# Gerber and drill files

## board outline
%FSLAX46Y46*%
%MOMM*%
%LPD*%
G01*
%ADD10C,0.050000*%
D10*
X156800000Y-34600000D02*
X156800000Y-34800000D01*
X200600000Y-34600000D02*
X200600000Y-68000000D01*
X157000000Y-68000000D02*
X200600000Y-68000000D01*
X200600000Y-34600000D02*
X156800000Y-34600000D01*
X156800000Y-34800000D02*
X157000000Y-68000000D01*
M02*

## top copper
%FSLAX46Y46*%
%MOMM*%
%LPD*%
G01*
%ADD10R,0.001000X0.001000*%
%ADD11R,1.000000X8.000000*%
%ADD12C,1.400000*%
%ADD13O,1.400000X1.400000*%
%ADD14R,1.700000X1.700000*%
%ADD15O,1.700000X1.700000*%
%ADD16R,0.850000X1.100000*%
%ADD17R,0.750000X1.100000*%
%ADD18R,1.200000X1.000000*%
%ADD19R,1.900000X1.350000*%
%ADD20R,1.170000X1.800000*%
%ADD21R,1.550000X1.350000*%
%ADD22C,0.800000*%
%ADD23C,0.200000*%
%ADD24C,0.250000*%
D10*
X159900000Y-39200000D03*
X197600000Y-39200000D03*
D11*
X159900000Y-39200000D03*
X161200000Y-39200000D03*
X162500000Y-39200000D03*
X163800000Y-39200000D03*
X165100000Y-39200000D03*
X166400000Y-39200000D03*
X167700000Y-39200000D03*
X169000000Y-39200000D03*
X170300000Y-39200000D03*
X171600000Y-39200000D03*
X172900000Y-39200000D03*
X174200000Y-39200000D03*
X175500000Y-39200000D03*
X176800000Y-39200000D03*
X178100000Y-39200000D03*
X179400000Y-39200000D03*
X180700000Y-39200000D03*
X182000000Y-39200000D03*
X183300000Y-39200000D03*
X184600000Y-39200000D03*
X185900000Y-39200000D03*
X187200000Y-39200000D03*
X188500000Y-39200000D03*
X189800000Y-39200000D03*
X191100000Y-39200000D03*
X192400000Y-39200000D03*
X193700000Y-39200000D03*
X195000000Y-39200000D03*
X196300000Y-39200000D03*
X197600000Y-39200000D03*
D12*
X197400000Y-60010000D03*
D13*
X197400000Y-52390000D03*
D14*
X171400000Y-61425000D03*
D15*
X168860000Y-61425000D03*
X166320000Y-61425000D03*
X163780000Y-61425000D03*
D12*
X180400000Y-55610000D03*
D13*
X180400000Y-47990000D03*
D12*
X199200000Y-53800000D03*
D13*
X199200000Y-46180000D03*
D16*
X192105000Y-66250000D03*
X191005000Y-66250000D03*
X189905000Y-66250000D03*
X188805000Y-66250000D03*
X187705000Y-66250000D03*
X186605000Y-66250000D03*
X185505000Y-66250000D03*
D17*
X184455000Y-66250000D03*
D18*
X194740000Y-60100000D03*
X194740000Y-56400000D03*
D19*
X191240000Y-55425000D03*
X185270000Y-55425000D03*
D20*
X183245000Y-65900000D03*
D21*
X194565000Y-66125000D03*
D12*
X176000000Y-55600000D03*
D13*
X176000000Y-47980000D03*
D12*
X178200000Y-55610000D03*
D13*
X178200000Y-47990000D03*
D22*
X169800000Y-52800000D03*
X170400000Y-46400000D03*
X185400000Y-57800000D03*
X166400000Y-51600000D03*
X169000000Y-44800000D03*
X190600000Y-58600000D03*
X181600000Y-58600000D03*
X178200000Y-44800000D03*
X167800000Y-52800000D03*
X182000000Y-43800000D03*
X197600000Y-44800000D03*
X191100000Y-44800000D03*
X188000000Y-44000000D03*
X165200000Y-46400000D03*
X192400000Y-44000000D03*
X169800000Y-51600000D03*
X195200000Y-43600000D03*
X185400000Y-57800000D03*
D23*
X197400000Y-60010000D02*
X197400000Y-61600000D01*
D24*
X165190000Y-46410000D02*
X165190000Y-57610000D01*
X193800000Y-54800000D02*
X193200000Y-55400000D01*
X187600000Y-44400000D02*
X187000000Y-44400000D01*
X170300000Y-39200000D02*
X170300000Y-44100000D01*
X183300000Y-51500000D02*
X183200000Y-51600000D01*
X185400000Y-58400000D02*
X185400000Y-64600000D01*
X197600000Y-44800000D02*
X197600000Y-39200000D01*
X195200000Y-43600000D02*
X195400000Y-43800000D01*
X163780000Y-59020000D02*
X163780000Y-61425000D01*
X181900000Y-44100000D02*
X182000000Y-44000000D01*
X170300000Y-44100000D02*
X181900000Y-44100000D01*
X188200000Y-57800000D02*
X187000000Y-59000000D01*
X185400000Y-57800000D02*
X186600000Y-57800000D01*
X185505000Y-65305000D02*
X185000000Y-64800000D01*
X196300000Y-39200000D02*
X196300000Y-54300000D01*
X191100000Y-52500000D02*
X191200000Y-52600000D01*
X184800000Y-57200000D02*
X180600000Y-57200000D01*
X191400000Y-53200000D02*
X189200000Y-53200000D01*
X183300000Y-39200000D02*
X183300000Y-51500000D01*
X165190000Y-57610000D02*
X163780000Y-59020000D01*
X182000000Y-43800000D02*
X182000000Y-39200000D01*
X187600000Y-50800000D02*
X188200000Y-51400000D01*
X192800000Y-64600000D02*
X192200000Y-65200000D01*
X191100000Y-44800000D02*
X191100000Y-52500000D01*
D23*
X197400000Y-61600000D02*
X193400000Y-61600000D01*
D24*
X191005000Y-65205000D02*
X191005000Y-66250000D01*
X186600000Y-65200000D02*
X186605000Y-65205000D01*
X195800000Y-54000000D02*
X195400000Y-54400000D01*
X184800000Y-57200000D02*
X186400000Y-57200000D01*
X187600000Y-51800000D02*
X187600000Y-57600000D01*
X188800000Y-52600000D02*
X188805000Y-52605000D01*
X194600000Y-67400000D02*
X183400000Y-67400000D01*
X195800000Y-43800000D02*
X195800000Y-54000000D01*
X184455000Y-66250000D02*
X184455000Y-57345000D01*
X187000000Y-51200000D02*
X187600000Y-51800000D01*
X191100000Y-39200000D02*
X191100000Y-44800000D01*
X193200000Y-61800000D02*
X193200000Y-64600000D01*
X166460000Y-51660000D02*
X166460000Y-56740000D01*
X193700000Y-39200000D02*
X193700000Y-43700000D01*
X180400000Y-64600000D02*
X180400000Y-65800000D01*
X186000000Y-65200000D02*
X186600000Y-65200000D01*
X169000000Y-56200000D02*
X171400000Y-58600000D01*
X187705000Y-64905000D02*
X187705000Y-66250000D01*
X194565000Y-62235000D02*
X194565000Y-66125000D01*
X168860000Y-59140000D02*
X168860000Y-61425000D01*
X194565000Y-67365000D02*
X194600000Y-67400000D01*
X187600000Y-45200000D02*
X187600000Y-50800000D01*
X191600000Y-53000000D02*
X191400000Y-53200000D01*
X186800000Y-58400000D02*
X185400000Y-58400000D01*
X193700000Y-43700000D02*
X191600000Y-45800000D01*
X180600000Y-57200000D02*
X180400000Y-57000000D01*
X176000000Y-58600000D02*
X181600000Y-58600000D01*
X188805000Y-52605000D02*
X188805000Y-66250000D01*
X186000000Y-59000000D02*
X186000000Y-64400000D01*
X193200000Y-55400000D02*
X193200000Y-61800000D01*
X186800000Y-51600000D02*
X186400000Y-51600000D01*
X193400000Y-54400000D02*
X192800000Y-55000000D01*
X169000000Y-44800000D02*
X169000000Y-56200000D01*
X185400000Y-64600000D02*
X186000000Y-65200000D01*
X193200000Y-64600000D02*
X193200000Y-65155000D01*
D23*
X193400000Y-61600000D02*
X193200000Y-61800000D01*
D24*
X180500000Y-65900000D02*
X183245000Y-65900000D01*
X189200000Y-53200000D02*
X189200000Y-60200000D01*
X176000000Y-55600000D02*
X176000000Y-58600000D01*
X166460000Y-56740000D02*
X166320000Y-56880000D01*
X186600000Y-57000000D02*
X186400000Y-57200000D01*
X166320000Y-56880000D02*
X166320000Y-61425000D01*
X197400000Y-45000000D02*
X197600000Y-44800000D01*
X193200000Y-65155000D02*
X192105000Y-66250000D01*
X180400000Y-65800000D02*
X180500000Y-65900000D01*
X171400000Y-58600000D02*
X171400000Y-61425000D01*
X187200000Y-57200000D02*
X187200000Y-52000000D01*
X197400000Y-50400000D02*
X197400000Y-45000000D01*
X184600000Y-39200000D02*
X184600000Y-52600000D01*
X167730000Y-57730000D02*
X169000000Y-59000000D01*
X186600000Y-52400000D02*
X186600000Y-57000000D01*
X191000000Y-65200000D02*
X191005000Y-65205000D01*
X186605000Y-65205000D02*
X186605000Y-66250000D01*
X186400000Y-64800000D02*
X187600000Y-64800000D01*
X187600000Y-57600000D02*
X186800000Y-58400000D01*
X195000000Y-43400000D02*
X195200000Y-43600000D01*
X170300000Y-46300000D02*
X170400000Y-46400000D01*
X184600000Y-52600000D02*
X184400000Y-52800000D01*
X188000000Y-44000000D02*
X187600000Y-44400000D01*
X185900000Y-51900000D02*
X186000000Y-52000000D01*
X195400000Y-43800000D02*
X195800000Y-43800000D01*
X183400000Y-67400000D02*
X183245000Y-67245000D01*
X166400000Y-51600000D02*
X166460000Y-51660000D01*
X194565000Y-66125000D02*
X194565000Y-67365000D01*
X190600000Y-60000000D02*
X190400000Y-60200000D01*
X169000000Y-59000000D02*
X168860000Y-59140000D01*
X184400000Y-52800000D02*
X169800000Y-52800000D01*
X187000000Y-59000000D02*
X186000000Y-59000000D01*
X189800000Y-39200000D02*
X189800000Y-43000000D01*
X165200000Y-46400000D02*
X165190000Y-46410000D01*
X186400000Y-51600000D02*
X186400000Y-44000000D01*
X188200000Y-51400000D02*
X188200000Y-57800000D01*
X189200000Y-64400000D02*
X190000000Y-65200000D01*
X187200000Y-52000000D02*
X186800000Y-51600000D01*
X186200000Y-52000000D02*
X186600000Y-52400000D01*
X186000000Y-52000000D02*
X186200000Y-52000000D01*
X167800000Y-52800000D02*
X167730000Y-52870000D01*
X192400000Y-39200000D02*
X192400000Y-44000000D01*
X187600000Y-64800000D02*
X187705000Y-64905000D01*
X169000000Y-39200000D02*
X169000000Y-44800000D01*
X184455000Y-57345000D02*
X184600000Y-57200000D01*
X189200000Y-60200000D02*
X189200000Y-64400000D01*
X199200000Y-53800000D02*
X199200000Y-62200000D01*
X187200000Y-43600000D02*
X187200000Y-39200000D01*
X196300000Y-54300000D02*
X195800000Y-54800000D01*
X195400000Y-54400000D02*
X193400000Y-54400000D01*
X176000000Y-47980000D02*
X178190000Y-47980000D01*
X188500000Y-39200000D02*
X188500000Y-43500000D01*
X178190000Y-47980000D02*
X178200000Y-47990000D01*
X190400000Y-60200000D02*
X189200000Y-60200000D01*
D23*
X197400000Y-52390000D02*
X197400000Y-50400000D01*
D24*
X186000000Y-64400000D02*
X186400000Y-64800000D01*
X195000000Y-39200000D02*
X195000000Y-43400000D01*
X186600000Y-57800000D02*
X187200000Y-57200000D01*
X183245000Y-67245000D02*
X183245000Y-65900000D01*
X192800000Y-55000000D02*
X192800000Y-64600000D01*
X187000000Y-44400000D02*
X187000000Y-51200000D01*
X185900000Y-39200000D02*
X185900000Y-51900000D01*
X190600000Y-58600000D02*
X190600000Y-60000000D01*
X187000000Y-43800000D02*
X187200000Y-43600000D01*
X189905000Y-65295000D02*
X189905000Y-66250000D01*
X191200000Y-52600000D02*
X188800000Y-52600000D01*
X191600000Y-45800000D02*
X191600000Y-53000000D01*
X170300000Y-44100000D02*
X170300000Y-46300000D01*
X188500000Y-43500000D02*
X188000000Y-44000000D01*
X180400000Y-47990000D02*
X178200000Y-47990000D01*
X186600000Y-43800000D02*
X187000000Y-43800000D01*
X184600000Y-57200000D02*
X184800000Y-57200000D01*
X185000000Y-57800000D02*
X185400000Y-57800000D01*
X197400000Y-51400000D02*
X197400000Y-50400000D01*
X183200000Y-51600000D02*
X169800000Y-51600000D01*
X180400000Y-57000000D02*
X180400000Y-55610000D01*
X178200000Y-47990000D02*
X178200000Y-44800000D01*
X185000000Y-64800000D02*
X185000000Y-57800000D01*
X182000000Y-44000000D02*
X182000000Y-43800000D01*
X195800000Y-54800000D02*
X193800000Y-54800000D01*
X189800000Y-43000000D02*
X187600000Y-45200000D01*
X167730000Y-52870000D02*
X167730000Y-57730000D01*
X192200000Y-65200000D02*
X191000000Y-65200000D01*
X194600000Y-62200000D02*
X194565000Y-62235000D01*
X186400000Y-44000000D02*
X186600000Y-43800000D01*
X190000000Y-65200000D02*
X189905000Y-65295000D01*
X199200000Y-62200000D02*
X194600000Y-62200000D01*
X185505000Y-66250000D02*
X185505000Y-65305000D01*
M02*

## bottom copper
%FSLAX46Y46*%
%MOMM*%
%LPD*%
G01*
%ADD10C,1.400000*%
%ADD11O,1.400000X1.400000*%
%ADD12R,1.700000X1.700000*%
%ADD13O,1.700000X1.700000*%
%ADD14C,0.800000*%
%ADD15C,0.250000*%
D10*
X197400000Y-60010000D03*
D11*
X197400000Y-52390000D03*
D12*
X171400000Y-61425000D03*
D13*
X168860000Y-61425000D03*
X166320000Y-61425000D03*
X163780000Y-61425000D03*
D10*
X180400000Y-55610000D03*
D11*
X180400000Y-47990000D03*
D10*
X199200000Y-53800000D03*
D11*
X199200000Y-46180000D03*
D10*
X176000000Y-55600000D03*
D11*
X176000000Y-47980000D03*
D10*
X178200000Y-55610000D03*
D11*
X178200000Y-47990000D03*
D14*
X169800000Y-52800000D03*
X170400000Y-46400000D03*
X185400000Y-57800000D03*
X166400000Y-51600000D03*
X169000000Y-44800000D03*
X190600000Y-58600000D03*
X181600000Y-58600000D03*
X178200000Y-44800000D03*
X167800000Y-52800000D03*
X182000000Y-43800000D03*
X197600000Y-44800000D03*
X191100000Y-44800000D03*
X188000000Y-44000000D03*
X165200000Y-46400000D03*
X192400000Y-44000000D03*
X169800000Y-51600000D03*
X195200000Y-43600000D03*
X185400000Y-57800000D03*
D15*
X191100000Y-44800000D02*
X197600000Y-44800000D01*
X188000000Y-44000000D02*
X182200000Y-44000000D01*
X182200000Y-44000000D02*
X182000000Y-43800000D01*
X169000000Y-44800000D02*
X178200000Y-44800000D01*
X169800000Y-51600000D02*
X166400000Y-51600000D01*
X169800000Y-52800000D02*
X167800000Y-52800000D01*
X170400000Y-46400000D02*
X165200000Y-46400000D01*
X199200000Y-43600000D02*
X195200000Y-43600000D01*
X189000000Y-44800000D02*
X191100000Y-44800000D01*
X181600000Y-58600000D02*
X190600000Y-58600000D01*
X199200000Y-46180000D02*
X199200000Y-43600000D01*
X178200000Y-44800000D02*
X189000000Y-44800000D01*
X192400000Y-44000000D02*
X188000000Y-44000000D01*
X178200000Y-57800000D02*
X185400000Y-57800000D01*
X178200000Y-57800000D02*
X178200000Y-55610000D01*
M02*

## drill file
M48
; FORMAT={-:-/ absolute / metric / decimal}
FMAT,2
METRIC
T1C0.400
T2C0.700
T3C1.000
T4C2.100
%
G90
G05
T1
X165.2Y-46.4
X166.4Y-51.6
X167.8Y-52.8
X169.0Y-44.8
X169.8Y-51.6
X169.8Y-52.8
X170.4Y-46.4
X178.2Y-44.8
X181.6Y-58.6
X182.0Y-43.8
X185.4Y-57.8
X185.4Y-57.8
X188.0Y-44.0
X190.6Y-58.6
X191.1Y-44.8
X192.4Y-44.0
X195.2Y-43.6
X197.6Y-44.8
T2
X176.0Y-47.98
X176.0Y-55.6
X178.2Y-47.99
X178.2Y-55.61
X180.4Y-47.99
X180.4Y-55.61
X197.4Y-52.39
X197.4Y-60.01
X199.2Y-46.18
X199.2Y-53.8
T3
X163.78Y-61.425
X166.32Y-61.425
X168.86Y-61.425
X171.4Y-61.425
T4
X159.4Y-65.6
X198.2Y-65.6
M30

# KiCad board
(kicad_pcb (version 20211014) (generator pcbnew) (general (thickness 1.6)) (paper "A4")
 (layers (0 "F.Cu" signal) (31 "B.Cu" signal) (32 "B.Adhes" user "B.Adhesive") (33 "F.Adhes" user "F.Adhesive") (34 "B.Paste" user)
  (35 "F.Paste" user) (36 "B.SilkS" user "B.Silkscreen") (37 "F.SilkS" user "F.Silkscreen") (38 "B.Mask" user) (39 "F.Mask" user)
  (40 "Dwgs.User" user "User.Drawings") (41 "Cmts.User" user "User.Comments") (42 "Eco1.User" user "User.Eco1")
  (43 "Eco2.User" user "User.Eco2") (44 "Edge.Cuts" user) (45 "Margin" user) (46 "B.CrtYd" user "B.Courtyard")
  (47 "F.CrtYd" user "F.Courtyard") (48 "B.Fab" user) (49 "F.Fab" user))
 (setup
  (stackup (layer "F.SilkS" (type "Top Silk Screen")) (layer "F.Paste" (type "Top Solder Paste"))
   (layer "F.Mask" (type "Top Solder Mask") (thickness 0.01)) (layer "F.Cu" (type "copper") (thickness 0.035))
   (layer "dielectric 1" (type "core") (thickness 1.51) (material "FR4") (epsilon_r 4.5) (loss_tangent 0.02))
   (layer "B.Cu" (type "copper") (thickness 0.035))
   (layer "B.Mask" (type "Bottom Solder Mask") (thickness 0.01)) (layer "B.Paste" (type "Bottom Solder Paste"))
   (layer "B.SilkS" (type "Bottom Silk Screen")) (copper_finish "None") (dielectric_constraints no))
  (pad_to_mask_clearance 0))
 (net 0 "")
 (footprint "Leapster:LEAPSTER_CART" (layer "F.Cu") (at 178.75 39.2)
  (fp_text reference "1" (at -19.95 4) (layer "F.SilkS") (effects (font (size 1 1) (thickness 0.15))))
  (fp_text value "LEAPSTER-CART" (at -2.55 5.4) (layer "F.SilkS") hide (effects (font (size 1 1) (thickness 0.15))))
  (pad "0" smd rect locked (at -18.85 0) (size 0.001 0.001) (layers "F.Cu" "F.Paste" "F.Mask"))
  (pad "0" smd rect locked (at 18.85 0) (size 0.001 0.001) (layers "F.Cu" "F.Paste" "F.Mask"))
  (pad "1" connect rect locked (at -18.85 0) (size 1 8) (layers "F.Cu" "F.Mask"))
  (pad "2" connect rect locked (at -17.55 0) (size 1 8) (layers "F.Cu" "F.Mask"))
  (pad "3" connect rect locked (at -16.25 0) (size 1 8) (layers "F.Cu" "F.Mask"))
  (pad "4" connect rect locked (at -14.95 0) (size 1 8) (layers "F.Cu" "F.Mask"))
  (pad "5" connect rect locked (at -13.65 0) (size 1 8) (layers "F.Cu" "F.Mask"))
  (pad "6" connect rect locked (at -12.35 0) (size 1 8) (layers "F.Cu" "F.Mask"))
  (pad "7" connect rect locked (at -11.05 0) (size 1 8) (layers "F.Cu" "F.Mask"))
  (pad "8" connect rect locked (at -9.75 0) (size 1 8) (layers "F.Cu" "F.Mask"))
  (pad "9" connect rect locked (at -8.45 0) (size 1 8) (layers "F.Cu" "F.Mask"))
  (pad "10" connect rect locked (at -7.15 0) (size 1 8) (layers "F.Cu" "F.Mask"))
  (pad "11" connect rect locked (at -5.85 0) (size 1 8) (layers "F.Cu" "F.Mask"))
  (pad "12" connect rect locked (at -4.55 0) (size 1 8) (layers "F.Cu" "F.Mask"))
  (pad "13" connect rect locked (at -3.25 0) (size 1 8) (layers "F.Cu" "F.Mask"))
  (pad "14" connect rect locked (at -1.95 0) (size 1 8) (layers "F.Cu" "F.Mask"))
  (pad "15" connect rect locked (at -0.65 0) (size 1 8) (layers "F.Cu" "F.Mask"))
  (pad "16" connect rect locked (at 0.65 0) (size 1 8) (layers "F.Cu" "F.Mask"))
  (pad "17" connect rect locked (at 1.95 0) (size 1 8) (layers "F.Cu" "F.Mask"))
  (pad "18" connect rect locked (at 3.25 0) (size 1 8) (layers "F.Cu" "F.Mask"))
  (pad "19" connect rect locked (at 4.55 0) (size 1 8) (layers "F.Cu" "F.Mask"))
  (pad "20" connect rect locked (at 5.85 0) (size 1 8) (layers "F.Cu" "F.Mask"))
  (pad "21" connect rect locked (at 7.15 0) (size 1 8) (layers "F.Cu" "F.Mask"))
  (pad "22" connect rect locked (at 8.45 0) (size 1 8) (layers "F.Cu" "F.Mask"))
  (pad "23" connect rect locked (at 9.75 0) (size 1 8) (layers "F.Cu" "F.Mask"))
  (pad "24" connect rect locked (at 11.05 0) (size 1 8) (layers "F.Cu" "F.Mask"))
  (pad "25" connect rect locked (at 12.35 0) (size 1 8) (layers "F.Cu" "F.Mask"))
  (pad "26" connect rect locked (at 13.65 0) (size 1 8) (layers "F.Cu" "F.Mask"))
  (pad "27" connect rect locked (at 14.95 0) (size 1 8) (layers "F.Cu" "F.Mask"))
  (pad "28" connect rect locked (at 16.25 0) (size 1 8) (layers "F.Cu" "F.Mask"))
  (pad "29" connect rect locked (at 17.55 0) (size 1 8) (layers "F.Cu" "F.Mask"))
  (pad "30" connect rect locked (at 18.85 0) (size 1 8) (layers "F.Cu" "F.Mask")))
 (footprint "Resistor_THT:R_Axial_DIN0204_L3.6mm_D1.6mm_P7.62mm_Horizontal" (layer "F.Cu") (at 197.4 60.01 90)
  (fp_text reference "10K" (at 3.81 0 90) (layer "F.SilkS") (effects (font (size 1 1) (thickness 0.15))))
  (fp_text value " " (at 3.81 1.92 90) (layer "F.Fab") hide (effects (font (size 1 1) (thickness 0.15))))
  (pad "1" thru_hole circle (at 0 0 90) (size 1.4 1.4) (drill 0.7) (layers *.Cu *.Mask))
  (pad "2" thru_hole oval (at 7.62 0 90) (size 1.4 1.4) (drill 0.7) (layers *.Cu *.Mask)))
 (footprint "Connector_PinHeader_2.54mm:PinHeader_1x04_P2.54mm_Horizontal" (layer "F.Cu") (at 171.4 61.425 -90)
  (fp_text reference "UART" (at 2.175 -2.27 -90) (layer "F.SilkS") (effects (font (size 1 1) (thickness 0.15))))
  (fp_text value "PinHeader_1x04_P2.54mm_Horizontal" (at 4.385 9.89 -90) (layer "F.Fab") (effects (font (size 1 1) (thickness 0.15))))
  (pad "1" thru_hole rect (at 0 0 270) (size 1.7 1.7) (drill 1) (layers *.Cu *.Mask))
  (pad "2" thru_hole oval (at 0 2.54 270) (size 1.7 1.7) (drill 1) (layers *.Cu *.Mask))
  (pad "3" thru_hole oval (at 0 5.08 270) (size 1.7 1.7) (drill 1) (layers *.Cu *.Mask))
  (pad "4" thru_hole oval (at 0 7.62 270) (size 1.7 1.7) (drill 1) (layers *.Cu *.Mask)))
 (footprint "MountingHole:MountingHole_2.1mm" (layer "F.Cu") (at 198.2 65.6)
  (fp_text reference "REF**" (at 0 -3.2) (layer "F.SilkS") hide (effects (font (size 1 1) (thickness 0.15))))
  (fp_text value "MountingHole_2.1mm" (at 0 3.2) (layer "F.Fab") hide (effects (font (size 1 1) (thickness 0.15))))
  (pad "" np_thru_hole circle (at 0 0) (size 1.5 1.5) (drill 2.1) (layers F&B.Cu *.Mask)))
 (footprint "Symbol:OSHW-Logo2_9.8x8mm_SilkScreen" (layer "F.Cu") (at 178 63)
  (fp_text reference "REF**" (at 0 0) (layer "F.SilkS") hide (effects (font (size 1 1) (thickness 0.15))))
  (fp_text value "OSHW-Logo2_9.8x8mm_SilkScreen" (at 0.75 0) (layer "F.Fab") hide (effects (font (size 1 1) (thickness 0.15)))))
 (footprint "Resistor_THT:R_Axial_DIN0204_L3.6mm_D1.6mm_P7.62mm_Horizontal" (layer "F.Cu") (at 180.4 55.61 90)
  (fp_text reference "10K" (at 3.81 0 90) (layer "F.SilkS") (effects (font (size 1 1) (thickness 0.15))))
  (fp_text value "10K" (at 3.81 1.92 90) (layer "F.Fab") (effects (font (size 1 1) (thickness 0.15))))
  (pad "1" thru_hole circle (at 0 0 90) (size 1.4 1.4) (drill 0.7) (layers *.Cu *.Mask))
  (pad "2" thru_hole oval (at 7.62 0 90) (size 1.4 1.4) (drill 0.7) (layers *.Cu *.Mask)))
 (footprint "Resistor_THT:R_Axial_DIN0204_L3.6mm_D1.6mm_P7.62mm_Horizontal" (layer "F.Cu") (at 199.2 53.8 90)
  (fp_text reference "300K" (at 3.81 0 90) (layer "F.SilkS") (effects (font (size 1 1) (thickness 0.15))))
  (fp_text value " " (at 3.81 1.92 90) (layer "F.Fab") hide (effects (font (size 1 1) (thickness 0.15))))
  (pad "1" thru_hole circle (at 0 0 90) (size 1.4 1.4) (drill 0.7) (layers *.Cu *.Mask))
  (pad "2" thru_hole oval (at 7.62 0 90) (size 1.4 1.4) (drill 0.7) (layers *.Cu *.Mask)))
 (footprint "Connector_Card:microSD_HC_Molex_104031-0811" (layer "F.Cu") (at 189 60.8 180)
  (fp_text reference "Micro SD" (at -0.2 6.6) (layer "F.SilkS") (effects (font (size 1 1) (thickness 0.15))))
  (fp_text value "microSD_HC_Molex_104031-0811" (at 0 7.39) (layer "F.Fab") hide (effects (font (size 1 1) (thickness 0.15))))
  (pad "1" smd rect (at -3.105 -5.45 180) (size 0.85 1.1) (layers "F.Cu" "F.Paste" "F.Mask"))
  (pad "2" smd rect (at -2.005 -5.45 180) (size 0.85 1.1) (layers "F.Cu" "F.Paste" "F.Mask"))
  (pad "3" smd rect (at -0.905 -5.45 180) (size 0.85 1.1) (layers "F.Cu" "F.Paste" "F.Mask"))
  (pad "4" smd rect (at 0.195 -5.45 180) (size 0.85 1.1) (layers "F.Cu" "F.Paste" "F.Mask"))
  (pad "5" smd rect (at 1.295 -5.45 180) (size 0.85 1.1) (layers "F.Cu" "F.Paste" "F.Mask"))
  (pad "6" smd rect (at 2.395 -5.45 180) (size 0.85 1.1) (layers "F.Cu" "F.Paste" "F.Mask"))
  (pad "7" smd rect (at 3.495 -5.45 180) (size 0.85 1.1) (layers "F.Cu" "F.Paste" "F.Mask"))
  (pad "8" smd rect (at 4.545 -5.45 180) (size 0.75 1.1) (layers "F.Cu" "F.Paste" "F.Mask"))
  (pad "9" smd rect (at -5.74 0.7 180) (size 1.2 1) (layers "F.Cu" "F.Paste" "F.Mask"))
  (pad "10" smd rect (at -5.74 4.4 180) (size 1.2 1) (layers "F.Cu" "F.Paste" "F.Mask"))
  (pad "11" smd rect (at -2.24 5.375 180) (size 1.9 1.35) (layers "F.Cu" "F.Paste" "F.Mask"))
  (pad "11" smd rect (at 3.73 5.375 180) (size 1.9 1.35) (layers "F.Cu" "F.Paste" "F.Mask"))
  (pad "11" smd rect (at 5.755 -5.1 180) (size 1.17 1.8) (layers "F.Cu" "F.Paste" "F.Mask"))
  (pad "11" smd rect (at -5.565 -5.325 180) (size 1.55 1.35) (layers "F.Cu" "F.Paste" "F.Mask")))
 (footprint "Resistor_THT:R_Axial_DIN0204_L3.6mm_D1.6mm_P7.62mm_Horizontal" (layer "F.Cu") (at 176 55.6 90)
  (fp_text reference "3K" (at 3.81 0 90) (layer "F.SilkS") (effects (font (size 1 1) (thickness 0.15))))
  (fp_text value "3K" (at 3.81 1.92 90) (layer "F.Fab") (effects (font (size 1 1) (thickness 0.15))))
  (pad "1" thru_hole circle (at 0 0 90) (size 1.4 1.4) (drill 0.7) (layers *.Cu *.Mask))
  (pad "2" thru_hole oval (at 7.62 0 90) (size 1.4 1.4) (drill 0.7) (layers *.Cu *.Mask)))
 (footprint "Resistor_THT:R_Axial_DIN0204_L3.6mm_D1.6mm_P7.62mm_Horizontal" (layer "F.Cu") (at 178.2 55.61 90)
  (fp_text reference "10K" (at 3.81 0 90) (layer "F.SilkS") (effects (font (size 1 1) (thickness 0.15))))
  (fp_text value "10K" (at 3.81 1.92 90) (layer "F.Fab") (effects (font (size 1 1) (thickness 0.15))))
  (pad "1" thru_hole circle (at 0 0 90) (size 1.4 1.4) (drill 0.7) (layers *.Cu *.Mask))
  (pad "2" thru_hole oval (at 7.62 0 90) (size 1.4 1.4) (drill 0.7) (layers *.Cu *.Mask)))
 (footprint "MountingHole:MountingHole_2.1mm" (layer "F.Cu") (at 159.4 65.6)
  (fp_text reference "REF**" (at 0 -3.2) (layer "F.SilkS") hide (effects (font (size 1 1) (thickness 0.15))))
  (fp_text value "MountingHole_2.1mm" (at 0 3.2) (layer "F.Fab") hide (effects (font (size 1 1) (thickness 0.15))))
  (pad "" np_thru_hole circle (at 0 0) (size 1.5 1.5) (drill 2.1) (layers F&B.Cu *.Mask)))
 (gr_line (start 156.8 34.6) (end 156.8 34.8) (layer "Edge.Cuts") (width 0.05))
 (gr_line (start 200.6 34.6) (end 200.6 68) (layer "Edge.Cuts") (width 0.05))
 (gr_line (start 157 68) (end 200.6 68) (layer "Edge.Cuts") (width 0.05))
 (gr_line (start 200.6 34.6) (end 156.8 34.6) (layer "Edge.Cuts") (width 0.05))
 (gr_line (start 156.8 34.8) (end 157 68) (layer "Edge.Cuts") (width 0.05))
 (segment (start 197.4 60.01) (end 197.4 61.6) (width 0.2) (layer "F.Cu") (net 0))
 (segment (start 165.19 46.41) (end 165.19 57.61) (width 0.25) (layer "F.Cu") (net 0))
 (segment (start 193.8 54.8) (end 193.2 55.4) (width 0.25) (layer "F.Cu") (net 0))
 (segment (start 187.6 44.4) (end 187 44.4) (width 0.25) (layer "F.Cu") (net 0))
 (segment (start 170.3 39.2) (end 170.3 44.1) (width 0.25) (layer "F.Cu") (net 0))
 (segment (start 183.3 51.5) (end 183.2 51.6) (width 0.25) (layer "F.Cu") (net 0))
 (segment (start 185.4 58.4) (end 185.4 64.6) (width 0.25) (layer "F.Cu") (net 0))
 (segment (start 197.6 44.8) (end 197.6 39.2) (width 0.25) (layer "F.Cu") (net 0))
 (segment (start 195.2 43.6) (end 195.4 43.8) (width 0.25) (layer "F.Cu") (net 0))
 (segment (start 163.78 59.02) (end 163.78 61.425) (width 0.25) (layer "F.Cu") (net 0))
 (segment (start 181.9 44.1) (end 182 44) (width 0.25) (layer "F.Cu") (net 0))
 (segment (start 170.3 44.1) (end 181.9 44.1) (width 0.25) (layer "F.Cu") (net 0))
 (segment (start 188.2 57.8) (end 187 59) (width 0.25) (layer "F.Cu") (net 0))
 (segment (start 185.4 57.8) (end 186.6 57.8) (width 0.25) (layer "F.Cu") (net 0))
 (segment (start 185.505 65.305) (end 185 64.8) (width 0.25) (layer "F.Cu") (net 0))
 (segment (start 196.3 39.2) (end 196.3 54.3) (width 0.25) (layer "F.Cu") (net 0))
 (segment (start 191.1 52.5) (end 191.2 52.6) (width 0.25) (layer "F.Cu") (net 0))
 (segment (start 184.8 57.2) (end 180.6 57.2) (width 0.25) (layer "F.Cu") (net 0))
 (segment (start 191.4 53.2) (end 189.2 53.2) (width 0.25) (layer "F.Cu") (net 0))
 (segment (start 183.3 39.2) (end 183.3 51.5) (width 0.25) (layer "F.Cu") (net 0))
 (segment (start 165.19 57.61) (end 163.78 59.02) (width 0.25) (layer "F.Cu") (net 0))
 (segment (start 182 43.8) (end 182 39.2) (width 0.25) (layer "F.Cu") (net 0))
 (segment (start 187.6 50.8) (end 188.2 51.4) (width 0.25) (layer "F.Cu") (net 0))
 (segment (start 192.8 64.6) (end 192.2 65.2) (width 0.25) (layer "F.Cu") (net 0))
 (segment (start 191.1 44.8) (end 191.1 52.5) (width 0.25) (layer "F.Cu") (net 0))
 (segment (start 197.4 61.6) (end 193.4 61.6) (width 0.2) (layer "F.Cu") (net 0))
 (segment (start 191.005 65.205) (end 191.005 66.25) (width 0.25) (layer "F.Cu") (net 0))
 (segment (start 186.6 65.2) (end 186.605 65.205) (width 0.25) (layer "F.Cu") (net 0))
 (segment (start 195.8 54) (end 195.4 54.4) (width 0.25) (layer "F.Cu") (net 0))
 (segment (start 184.8 57.2) (end 186.4 57.2) (width 0.25) (layer "F.Cu") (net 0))
 (segment (start 187.6 51.8) (end 187.6 57.6) (width 0.25) (layer "F.Cu") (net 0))
 (segment (start 188.8 52.6) (end 188.805 52.605) (width 0.25) (layer "F.Cu") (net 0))
 (segment (start 194.6 67.4) (end 183.4 67.4) (width 0.25) (layer "F.Cu") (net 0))
 (segment (start 195.8 43.8) (end 195.8 54) (width 0.25) (layer "F.Cu") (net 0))
 (segment (start 184.455 66.25) (end 184.455 57.345) (width 0.25) (layer "F.Cu") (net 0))
 (segment (start 187 51.2) (end 187.6 51.8) (width 0.25) (layer "F.Cu") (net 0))
 (segment (start 191.1 39.2) (end 191.1 44.8) (width 0.25) (layer "F.Cu") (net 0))
 (segment (start 193.2 61.8) (end 193.2 64.6) (width 0.25) (layer "F.Cu") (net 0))
 (segment (start 166.46 51.66) (end 166.46 56.74) (width 0.25) (layer "F.Cu") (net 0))
 (segment (start 193.7 39.2) (end 193.7 43.7) (width 0.25) (layer "F.Cu") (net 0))
 (segment (start 180.4 64.6) (end 180.4 65.8) (width 0.25) (layer "F.Cu") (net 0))
 (segment (start 186 65.2) (end 186.6 65.2) (width 0.25) (layer "F.Cu") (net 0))
 (segment (start 169 56.2) (end 171.4 58.6) (width 0.25) (layer "F.Cu") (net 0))
 (segment (start 187.705 64.905) (end 187.705 66.25) (width 0.25) (layer "F.Cu") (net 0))
 (segment (start 194.565 62.235) (end 194.565 66.125) (width 0.25) (layer "F.Cu") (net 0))
 (segment (start 168.86 59.14) (end 168.86 61.425) (width 0.25) (layer "F.Cu") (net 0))
 (segment (start 194.565 67.365) (end 194.6 67.4) (width 0.25) (layer "F.Cu") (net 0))
 (segment (start 187.6 45.2) (end 187.6 50.8) (width 0.25) (layer "F.Cu") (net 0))
 (segment (start 191.6 53) (end 191.4 53.2) (width 0.25) (layer "F.Cu") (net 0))
 (segment (start 186.8 58.4) (end 185.4 58.4) (width 0.25) (layer "F.Cu") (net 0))
 (segment (start 193.7 43.7) (end 191.6 45.8) (width 0.25) (layer "F.Cu") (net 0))
 (segment (start 180.6 57.2) (end 180.4 57) (width 0.25) (layer "F.Cu") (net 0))
 (segment (start 176 58.6) (end 181.6 58.6) (width 0.25) (layer "F.Cu") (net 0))
 (segment (start 188.805 52.605) (end 188.805 66.25) (width 0.25) (layer "F.Cu") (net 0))
 (segment (start 186 59) (end 186 64.4) (width 0.25) (layer "F.Cu") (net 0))
 (segment (start 193.2 55.4) (end 193.2 61.8) (width 0.25) (layer "F.Cu") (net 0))
 (segment (start 186.8 51.6) (end 186.4 51.6) (width 0.25) (layer "F.Cu") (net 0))
 (segment (start 193.4 54.4) (end 192.8 55) (width 0.25) (layer "F.Cu") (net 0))
 (segment (start 169 44.8) (end 169 56.2) (width 0.25) (layer "F.Cu") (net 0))
 (segment (start 185.4 64.6) (end 186 65.2) (width 0.25) (layer "F.Cu") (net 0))
 (segment (start 193.2 64.6) (end 193.2 65.155) (width 0.25) (layer "F.Cu") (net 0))
 (segment (start 193.4 61.6) (end 193.2 61.8) (width 0.2) (layer "F.Cu") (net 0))
 (segment (start 180.5 65.9) (end 183.245 65.9) (width 0.25) (layer "F.Cu") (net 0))
 (segment (start 189.2 53.2) (end 189.2 60.2) (width 0.25) (layer "F.Cu") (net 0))
 (segment (start 176 55.6) (end 176 58.6) (width 0.25) (layer "F.Cu") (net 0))
 (segment (start 166.46 56.74) (end 166.32 56.88) (width 0.25) (layer "F.Cu") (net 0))
 (segment (start 186.6 57) (end 186.4 57.2) (width 0.25) (layer "F.Cu") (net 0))
 (segment (start 166.32 56.88) (end 166.32 61.425) (width 0.25) (layer "F.Cu") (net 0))
 (segment (start 197.4 45) (end 197.6 44.8) (width 0.25) (layer "F.Cu") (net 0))
 (segment (start 193.2 65.155) (end 192.105 66.25) (width 0.25) (layer "F.Cu") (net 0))
 (segment (start 180.4 65.8) (end 180.5 65.9) (width 0.25) (layer "F.Cu") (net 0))
 (segment (start 171.4 58.6) (end 171.4 61.425) (width 0.25) (layer "F.Cu") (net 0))
 (segment (start 187.2 57.2) (end 187.2 52) (width 0.25) (layer "F.Cu") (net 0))
 (segment (start 197.4 50.4) (end 197.4 45) (width 0.25) (layer "F.Cu") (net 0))
 (segment (start 184.6 39.2) (end 184.6 52.6) (width 0.25) (layer "F.Cu") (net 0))
 (segment (start 167.73 57.73) (end 169 59) (width 0.25) (layer "F.Cu") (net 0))
 (segment (start 186.6 52.4) (end 186.6 57) (width 0.25) (layer "F.Cu") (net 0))
 (segment (start 191 65.2) (end 191.005 65.205) (width 0.25) (layer "F.Cu") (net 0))
 (segment (start 186.605 65.205) (end 186.605 66.25) (width 0.25) (layer "F.Cu") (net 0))
 (segment (start 186.4 64.8) (end 187.6 64.8) (width 0.25) (layer "F.Cu") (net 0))
 (segment (start 187.6 57.6) (end 186.8 58.4) (width 0.25) (layer "F.Cu") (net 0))
 (segment (start 195 43.4) (end 195.2 43.6) (width 0.25) (layer "F.Cu") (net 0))
 (segment (start 170.3 46.3) (end 170.4 46.4) (width 0.25) (layer "F.Cu") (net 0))
 (segment (start 184.6 52.6) (end 184.4 52.8) (width 0.25) (layer "F.Cu") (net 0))
 (segment (start 188 44) (end 187.6 44.4) (width 0.25) (layer "F.Cu") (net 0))
 (segment (start 185.9 51.9) (end 186 52) (width 0.25) (layer "F.Cu") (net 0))
 (segment (start 195.4 43.8) (end 195.8 43.8) (width 0.25) (layer "F.Cu") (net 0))
 (segment (start 183.4 67.4) (end 183.245 67.245) (width 0.25) (layer "F.Cu") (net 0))
 (segment (start 166.4 51.6) (end 166.46 51.66) (width 0.25) (layer "F.Cu") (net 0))
 (segment (start 194.565 66.125) (end 194.565 67.365) (width 0.25) (layer "F.Cu") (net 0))
 (segment (start 190.6 60) (end 190.4 60.2) (width 0.25) (layer "F.Cu") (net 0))
 (segment (start 169 59) (end 168.86 59.14) (width 0.25) (layer "F.Cu") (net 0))
 (segment (start 184.4 52.8) (end 169.8 52.8) (width 0.25) (layer "F.Cu") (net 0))
 (segment (start 187 59) (end 186 59) (width 0.25) (layer "F.Cu") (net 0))
 (segment (start 189.8 39.2) (end 189.8 43) (width 0.25) (layer "F.Cu") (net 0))
 (segment (start 165.2 46.4) (end 165.19 46.41) (width 0.25) (layer "F.Cu") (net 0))
 (segment (start 186.4 51.6) (end 186.4 44) (width 0.25) (layer "F.Cu") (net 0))
 (segment (start 188.2 51.4) (end 188.2 57.8) (width 0.25) (layer "F.Cu") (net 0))
 (segment (start 189.2 64.4) (end 190 65.2) (width 0.25) (layer "F.Cu") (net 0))
 (segment (start 187.2 52) (end 186.8 51.6) (width 0.25) (layer "F.Cu") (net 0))
 (segment (start 186.2 52) (end 186.6 52.4) (width 0.25) (layer "F.Cu") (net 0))
 (segment (start 186 52) (end 186.2 52) (width 0.25) (layer "F.Cu") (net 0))
 (segment (start 167.8 52.8) (end 167.73 52.87) (width 0.25) (layer "F.Cu") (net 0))
 (segment (start 192.4 39.2) (end 192.4 44) (width 0.25) (layer "F.Cu") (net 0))
 (segment (start 187.6 64.8) (end 187.705 64.905) (width 0.25) (layer "F.Cu") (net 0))
 (segment (start 169 39.2) (end 169 44.8) (width 0.25) (layer "F.Cu") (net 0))
 (segment (start 184.455 57.345) (end 184.6 57.2) (width 0.25) (layer "F.Cu") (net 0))
 (segment (start 189.2 60.2) (end 189.2 64.4) (width 0.25) (layer "F.Cu") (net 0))
 (segment (start 199.2 53.8) (end 199.2 62.2) (width 0.25) (layer "F.Cu") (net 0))
 (segment (start 187.2 43.6) (end 187.2 39.2) (width 0.25) (layer "F.Cu") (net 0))
 (segment (start 196.3 54.3) (end 195.8 54.8) (width 0.25) (layer "F.Cu") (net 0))
 (segment (start 195.4 54.4) (end 193.4 54.4) (width 0.25) (layer "F.Cu") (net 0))
 (segment (start 176 47.98) (end 178.19 47.98) (width 0.25) (layer "F.Cu") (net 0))
 (segment (start 188.5 39.2) (end 188.5 43.5) (width 0.25) (layer "F.Cu") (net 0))
 (segment (start 178.19 47.98) (end 178.2 47.99) (width 0.25) (layer "F.Cu") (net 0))
 (segment (start 190.4 60.2) (end 189.2 60.2) (width 0.25) (layer "F.Cu") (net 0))
 (segment (start 197.4 52.39) (end 197.4 50.4) (width 0.2) (layer "F.Cu") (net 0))
 (segment (start 186 64.4) (end 186.4 64.8) (width 0.25) (layer "F.Cu") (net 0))
 (segment (start 195 39.2) (end 195 43.4) (width 0.25) (layer "F.Cu") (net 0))
 (segment (start 186.6 57.8) (end 187.2 57.2) (width 0.25) (layer "F.Cu") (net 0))
 (segment (start 183.245 67.245) (end 183.245 65.9) (width 0.25) (layer "F.Cu") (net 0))
 (segment (start 192.8 55) (end 192.8 64.6) (width 0.25) (layer "F.Cu") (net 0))
 (segment (start 187 44.4) (end 187 51.2) (width 0.25) (layer "F.Cu") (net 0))
 (segment (start 185.9 39.2) (end 185.9 51.9) (width 0.25) (layer "F.Cu") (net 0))
 (segment (start 190.6 58.6) (end 190.6 60) (width 0.25) (layer "F.Cu") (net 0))
 (segment (start 187 43.8) (end 187.2 43.6) (width 0.25) (layer "F.Cu") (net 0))
 (segment (start 189.905 65.295) (end 189.905 66.25) (width 0.25) (layer "F.Cu") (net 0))
 (segment (start 191.2 52.6) (end 188.8 52.6) (width 0.25) (layer "F.Cu") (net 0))
 (segment (start 191.6 45.8) (end 191.6 53) (width 0.25) (layer "F.Cu") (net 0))
 (segment (start 170.3 44.1) (end 170.3 46.3) (width 0.25) (layer "F.Cu") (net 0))
 (segment (start 188.5 43.5) (end 188 44) (width 0.25) (layer "F.Cu") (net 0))
 (segment (start 180.4 47.99) (end 178.2 47.99) (width 0.25) (layer "F.Cu") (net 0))
 (segment (start 186.6 43.8) (end 187 43.8) (width 0.25) (layer "F.Cu") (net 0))
 (segment (start 184.6 57.2) (end 184.8 57.2) (width 0.25) (layer "F.Cu") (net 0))
 (segment (start 185 57.8) (end 185.4 57.8) (width 0.25) (layer "F.Cu") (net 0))
 (segment (start 197.4 51.4) (end 197.4 50.4) (width 0.25) (layer "F.Cu") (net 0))
 (segment (start 183.2 51.6) (end 169.8 51.6) (width 0.25) (layer "F.Cu") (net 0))
 (segment (start 180.4 57) (end 180.4 55.61) (width 0.25) (layer "F.Cu") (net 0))
 (segment (start 178.2 47.99) (end 178.2 44.8) (width 0.25) (layer "F.Cu") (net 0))
 (segment (start 185 64.8) (end 185 57.8) (width 0.25) (layer "F.Cu") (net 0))
 (segment (start 182 44) (end 182 43.8) (width 0.25) (layer "F.Cu") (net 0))
 (segment (start 195.8 54.8) (end 193.8 54.8) (width 0.25) (layer "F.Cu") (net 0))
 (segment (start 189.8 43) (end 187.6 45.2) (width 0.25) (layer "F.Cu") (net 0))
 (segment (start 167.73 52.87) (end 167.73 57.73) (width 0.25) (layer "F.Cu") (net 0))
 (segment (start 192.2 65.2) (end 191 65.2) (width 0.25) (layer "F.Cu") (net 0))
 (segment (start 194.6 62.2) (end 194.565 62.235) (width 0.25) (layer "F.Cu") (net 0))
 (segment (start 186.4 44) (end 186.6 43.8) (width 0.25) (layer "F.Cu") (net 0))
 (segment (start 190 65.2) (end 189.905 65.295) (width 0.25) (layer "F.Cu") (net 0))
 (segment (start 199.2 62.2) (end 194.6 62.2) (width 0.25) (layer "F.Cu") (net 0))
 (segment (start 185.505 66.25) (end 185.505 65.305) (width 0.25) (layer "F.Cu") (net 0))
 (via (at 169.8 52.8) (size 0.8) (drill 0.4) (layers "F.Cu" "B.Cu") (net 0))
 (via (at 170.4 46.4) (size 0.8) (drill 0.4) (layers "F.Cu" "B.Cu") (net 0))
 (via (at 185.4 57.8) (size 0.8) (drill 0.4) (layers "F.Cu" "B.Cu") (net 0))
 (via (at 166.4 51.6) (size 0.8) (drill 0.4) (layers "F.Cu" "B.Cu") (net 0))
 (via (at 169 44.8) (size 0.8) (drill 0.4) (layers "F.Cu" "B.Cu") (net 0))
 (via (at 190.6 58.6) (size 0.8) (drill 0.4) (layers "F.Cu" "B.Cu") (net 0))
 (via (at 181.6 58.6) (size 0.8) (drill 0.4) (layers "F.Cu" "B.Cu") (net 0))
 (via (at 178.2 44.8) (size 0.8) (drill 0.4) (layers "F.Cu" "B.Cu") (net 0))
 (via (at 167.8 52.8) (size 0.8) (drill 0.4) (layers "F.Cu" "B.Cu") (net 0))
 (via (at 182 43.8) (size 0.8) (drill 0.4) (layers "F.Cu" "B.Cu") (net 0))
 (via (at 197.6 44.8) (size 0.8) (drill 0.4) (layers "F.Cu" "B.Cu") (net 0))
 (via (at 191.1 44.8) (size 0.8) (drill 0.4) (layers "F.Cu" "B.Cu") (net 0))
 (via (at 188 44) (size 0.8) (drill 0.4) (layers "F.Cu" "B.Cu") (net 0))
 (via (at 165.2 46.4) (size 0.8) (drill 0.4) (layers "F.Cu" "B.Cu") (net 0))
 (via (at 192.4 44) (size 0.8) (drill 0.4) (layers "F.Cu" "B.Cu") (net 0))
 (via (at 169.8 51.6) (size 0.8) (drill 0.4) (layers "F.Cu" "B.Cu") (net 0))
 (via (at 195.2 43.6) (size 0.8) (drill 0.4) (layers "F.Cu" "B.Cu") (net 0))
 (via (at 185.4 57.8) (size 0.8) (drill 0.4) (layers "F.Cu" "B.Cu") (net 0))
 (segment (start 191.1 44.8) (end 197.6 44.8) (width 0.25) (layer "B.Cu") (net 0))
 (segment (start 188 44) (end 182.2 44) (width 0.25) (layer "B.Cu") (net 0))
 (segment (start 182.2 44) (end 182 43.8) (width 0.25) (layer "B.Cu") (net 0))
 (segment (start 169 44.8) (end 178.2 44.8) (width 0.25) (layer "B.Cu") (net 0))
 (segment (start 169.8 51.6) (end 166.4 51.6) (width 0.25) (layer "B.Cu") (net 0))
 (segment (start 169.8 52.8) (end 167.8 52.8) (width 0.25) (layer "B.Cu") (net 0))
 (segment (start 170.4 46.4) (end 165.2 46.4) (width 0.25) (layer "B.Cu") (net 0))
 (segment (start 199.2 43.6) (end 195.2 43.6) (width 0.25) (layer "B.Cu") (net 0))
 (segment (start 189 44.8) (end 191.1 44.8) (width 0.25) (layer "B.Cu") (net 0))
 (segment (start 181.6 58.6) (end 190.6 58.6) (width 0.25) (layer "B.Cu") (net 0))
 (segment (start 199.2 46.18) (end 199.2 43.6) (width 0.25) (layer "B.Cu") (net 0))
 (segment (start 178.2 44.8) (end 189 44.8) (width 0.25) (layer "B.Cu") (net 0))
 (segment (start 192.4 44) (end 188 44) (width 0.25) (layer "B.Cu") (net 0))
 (segment (start 178.2 57.8) (end 185.4 57.8) (width 0.25) (layer "B.Cu") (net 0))
 (segment (start 178.2 57.8) (end 178.2 55.61) (width 0.25) (layer "B.Cu") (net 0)))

